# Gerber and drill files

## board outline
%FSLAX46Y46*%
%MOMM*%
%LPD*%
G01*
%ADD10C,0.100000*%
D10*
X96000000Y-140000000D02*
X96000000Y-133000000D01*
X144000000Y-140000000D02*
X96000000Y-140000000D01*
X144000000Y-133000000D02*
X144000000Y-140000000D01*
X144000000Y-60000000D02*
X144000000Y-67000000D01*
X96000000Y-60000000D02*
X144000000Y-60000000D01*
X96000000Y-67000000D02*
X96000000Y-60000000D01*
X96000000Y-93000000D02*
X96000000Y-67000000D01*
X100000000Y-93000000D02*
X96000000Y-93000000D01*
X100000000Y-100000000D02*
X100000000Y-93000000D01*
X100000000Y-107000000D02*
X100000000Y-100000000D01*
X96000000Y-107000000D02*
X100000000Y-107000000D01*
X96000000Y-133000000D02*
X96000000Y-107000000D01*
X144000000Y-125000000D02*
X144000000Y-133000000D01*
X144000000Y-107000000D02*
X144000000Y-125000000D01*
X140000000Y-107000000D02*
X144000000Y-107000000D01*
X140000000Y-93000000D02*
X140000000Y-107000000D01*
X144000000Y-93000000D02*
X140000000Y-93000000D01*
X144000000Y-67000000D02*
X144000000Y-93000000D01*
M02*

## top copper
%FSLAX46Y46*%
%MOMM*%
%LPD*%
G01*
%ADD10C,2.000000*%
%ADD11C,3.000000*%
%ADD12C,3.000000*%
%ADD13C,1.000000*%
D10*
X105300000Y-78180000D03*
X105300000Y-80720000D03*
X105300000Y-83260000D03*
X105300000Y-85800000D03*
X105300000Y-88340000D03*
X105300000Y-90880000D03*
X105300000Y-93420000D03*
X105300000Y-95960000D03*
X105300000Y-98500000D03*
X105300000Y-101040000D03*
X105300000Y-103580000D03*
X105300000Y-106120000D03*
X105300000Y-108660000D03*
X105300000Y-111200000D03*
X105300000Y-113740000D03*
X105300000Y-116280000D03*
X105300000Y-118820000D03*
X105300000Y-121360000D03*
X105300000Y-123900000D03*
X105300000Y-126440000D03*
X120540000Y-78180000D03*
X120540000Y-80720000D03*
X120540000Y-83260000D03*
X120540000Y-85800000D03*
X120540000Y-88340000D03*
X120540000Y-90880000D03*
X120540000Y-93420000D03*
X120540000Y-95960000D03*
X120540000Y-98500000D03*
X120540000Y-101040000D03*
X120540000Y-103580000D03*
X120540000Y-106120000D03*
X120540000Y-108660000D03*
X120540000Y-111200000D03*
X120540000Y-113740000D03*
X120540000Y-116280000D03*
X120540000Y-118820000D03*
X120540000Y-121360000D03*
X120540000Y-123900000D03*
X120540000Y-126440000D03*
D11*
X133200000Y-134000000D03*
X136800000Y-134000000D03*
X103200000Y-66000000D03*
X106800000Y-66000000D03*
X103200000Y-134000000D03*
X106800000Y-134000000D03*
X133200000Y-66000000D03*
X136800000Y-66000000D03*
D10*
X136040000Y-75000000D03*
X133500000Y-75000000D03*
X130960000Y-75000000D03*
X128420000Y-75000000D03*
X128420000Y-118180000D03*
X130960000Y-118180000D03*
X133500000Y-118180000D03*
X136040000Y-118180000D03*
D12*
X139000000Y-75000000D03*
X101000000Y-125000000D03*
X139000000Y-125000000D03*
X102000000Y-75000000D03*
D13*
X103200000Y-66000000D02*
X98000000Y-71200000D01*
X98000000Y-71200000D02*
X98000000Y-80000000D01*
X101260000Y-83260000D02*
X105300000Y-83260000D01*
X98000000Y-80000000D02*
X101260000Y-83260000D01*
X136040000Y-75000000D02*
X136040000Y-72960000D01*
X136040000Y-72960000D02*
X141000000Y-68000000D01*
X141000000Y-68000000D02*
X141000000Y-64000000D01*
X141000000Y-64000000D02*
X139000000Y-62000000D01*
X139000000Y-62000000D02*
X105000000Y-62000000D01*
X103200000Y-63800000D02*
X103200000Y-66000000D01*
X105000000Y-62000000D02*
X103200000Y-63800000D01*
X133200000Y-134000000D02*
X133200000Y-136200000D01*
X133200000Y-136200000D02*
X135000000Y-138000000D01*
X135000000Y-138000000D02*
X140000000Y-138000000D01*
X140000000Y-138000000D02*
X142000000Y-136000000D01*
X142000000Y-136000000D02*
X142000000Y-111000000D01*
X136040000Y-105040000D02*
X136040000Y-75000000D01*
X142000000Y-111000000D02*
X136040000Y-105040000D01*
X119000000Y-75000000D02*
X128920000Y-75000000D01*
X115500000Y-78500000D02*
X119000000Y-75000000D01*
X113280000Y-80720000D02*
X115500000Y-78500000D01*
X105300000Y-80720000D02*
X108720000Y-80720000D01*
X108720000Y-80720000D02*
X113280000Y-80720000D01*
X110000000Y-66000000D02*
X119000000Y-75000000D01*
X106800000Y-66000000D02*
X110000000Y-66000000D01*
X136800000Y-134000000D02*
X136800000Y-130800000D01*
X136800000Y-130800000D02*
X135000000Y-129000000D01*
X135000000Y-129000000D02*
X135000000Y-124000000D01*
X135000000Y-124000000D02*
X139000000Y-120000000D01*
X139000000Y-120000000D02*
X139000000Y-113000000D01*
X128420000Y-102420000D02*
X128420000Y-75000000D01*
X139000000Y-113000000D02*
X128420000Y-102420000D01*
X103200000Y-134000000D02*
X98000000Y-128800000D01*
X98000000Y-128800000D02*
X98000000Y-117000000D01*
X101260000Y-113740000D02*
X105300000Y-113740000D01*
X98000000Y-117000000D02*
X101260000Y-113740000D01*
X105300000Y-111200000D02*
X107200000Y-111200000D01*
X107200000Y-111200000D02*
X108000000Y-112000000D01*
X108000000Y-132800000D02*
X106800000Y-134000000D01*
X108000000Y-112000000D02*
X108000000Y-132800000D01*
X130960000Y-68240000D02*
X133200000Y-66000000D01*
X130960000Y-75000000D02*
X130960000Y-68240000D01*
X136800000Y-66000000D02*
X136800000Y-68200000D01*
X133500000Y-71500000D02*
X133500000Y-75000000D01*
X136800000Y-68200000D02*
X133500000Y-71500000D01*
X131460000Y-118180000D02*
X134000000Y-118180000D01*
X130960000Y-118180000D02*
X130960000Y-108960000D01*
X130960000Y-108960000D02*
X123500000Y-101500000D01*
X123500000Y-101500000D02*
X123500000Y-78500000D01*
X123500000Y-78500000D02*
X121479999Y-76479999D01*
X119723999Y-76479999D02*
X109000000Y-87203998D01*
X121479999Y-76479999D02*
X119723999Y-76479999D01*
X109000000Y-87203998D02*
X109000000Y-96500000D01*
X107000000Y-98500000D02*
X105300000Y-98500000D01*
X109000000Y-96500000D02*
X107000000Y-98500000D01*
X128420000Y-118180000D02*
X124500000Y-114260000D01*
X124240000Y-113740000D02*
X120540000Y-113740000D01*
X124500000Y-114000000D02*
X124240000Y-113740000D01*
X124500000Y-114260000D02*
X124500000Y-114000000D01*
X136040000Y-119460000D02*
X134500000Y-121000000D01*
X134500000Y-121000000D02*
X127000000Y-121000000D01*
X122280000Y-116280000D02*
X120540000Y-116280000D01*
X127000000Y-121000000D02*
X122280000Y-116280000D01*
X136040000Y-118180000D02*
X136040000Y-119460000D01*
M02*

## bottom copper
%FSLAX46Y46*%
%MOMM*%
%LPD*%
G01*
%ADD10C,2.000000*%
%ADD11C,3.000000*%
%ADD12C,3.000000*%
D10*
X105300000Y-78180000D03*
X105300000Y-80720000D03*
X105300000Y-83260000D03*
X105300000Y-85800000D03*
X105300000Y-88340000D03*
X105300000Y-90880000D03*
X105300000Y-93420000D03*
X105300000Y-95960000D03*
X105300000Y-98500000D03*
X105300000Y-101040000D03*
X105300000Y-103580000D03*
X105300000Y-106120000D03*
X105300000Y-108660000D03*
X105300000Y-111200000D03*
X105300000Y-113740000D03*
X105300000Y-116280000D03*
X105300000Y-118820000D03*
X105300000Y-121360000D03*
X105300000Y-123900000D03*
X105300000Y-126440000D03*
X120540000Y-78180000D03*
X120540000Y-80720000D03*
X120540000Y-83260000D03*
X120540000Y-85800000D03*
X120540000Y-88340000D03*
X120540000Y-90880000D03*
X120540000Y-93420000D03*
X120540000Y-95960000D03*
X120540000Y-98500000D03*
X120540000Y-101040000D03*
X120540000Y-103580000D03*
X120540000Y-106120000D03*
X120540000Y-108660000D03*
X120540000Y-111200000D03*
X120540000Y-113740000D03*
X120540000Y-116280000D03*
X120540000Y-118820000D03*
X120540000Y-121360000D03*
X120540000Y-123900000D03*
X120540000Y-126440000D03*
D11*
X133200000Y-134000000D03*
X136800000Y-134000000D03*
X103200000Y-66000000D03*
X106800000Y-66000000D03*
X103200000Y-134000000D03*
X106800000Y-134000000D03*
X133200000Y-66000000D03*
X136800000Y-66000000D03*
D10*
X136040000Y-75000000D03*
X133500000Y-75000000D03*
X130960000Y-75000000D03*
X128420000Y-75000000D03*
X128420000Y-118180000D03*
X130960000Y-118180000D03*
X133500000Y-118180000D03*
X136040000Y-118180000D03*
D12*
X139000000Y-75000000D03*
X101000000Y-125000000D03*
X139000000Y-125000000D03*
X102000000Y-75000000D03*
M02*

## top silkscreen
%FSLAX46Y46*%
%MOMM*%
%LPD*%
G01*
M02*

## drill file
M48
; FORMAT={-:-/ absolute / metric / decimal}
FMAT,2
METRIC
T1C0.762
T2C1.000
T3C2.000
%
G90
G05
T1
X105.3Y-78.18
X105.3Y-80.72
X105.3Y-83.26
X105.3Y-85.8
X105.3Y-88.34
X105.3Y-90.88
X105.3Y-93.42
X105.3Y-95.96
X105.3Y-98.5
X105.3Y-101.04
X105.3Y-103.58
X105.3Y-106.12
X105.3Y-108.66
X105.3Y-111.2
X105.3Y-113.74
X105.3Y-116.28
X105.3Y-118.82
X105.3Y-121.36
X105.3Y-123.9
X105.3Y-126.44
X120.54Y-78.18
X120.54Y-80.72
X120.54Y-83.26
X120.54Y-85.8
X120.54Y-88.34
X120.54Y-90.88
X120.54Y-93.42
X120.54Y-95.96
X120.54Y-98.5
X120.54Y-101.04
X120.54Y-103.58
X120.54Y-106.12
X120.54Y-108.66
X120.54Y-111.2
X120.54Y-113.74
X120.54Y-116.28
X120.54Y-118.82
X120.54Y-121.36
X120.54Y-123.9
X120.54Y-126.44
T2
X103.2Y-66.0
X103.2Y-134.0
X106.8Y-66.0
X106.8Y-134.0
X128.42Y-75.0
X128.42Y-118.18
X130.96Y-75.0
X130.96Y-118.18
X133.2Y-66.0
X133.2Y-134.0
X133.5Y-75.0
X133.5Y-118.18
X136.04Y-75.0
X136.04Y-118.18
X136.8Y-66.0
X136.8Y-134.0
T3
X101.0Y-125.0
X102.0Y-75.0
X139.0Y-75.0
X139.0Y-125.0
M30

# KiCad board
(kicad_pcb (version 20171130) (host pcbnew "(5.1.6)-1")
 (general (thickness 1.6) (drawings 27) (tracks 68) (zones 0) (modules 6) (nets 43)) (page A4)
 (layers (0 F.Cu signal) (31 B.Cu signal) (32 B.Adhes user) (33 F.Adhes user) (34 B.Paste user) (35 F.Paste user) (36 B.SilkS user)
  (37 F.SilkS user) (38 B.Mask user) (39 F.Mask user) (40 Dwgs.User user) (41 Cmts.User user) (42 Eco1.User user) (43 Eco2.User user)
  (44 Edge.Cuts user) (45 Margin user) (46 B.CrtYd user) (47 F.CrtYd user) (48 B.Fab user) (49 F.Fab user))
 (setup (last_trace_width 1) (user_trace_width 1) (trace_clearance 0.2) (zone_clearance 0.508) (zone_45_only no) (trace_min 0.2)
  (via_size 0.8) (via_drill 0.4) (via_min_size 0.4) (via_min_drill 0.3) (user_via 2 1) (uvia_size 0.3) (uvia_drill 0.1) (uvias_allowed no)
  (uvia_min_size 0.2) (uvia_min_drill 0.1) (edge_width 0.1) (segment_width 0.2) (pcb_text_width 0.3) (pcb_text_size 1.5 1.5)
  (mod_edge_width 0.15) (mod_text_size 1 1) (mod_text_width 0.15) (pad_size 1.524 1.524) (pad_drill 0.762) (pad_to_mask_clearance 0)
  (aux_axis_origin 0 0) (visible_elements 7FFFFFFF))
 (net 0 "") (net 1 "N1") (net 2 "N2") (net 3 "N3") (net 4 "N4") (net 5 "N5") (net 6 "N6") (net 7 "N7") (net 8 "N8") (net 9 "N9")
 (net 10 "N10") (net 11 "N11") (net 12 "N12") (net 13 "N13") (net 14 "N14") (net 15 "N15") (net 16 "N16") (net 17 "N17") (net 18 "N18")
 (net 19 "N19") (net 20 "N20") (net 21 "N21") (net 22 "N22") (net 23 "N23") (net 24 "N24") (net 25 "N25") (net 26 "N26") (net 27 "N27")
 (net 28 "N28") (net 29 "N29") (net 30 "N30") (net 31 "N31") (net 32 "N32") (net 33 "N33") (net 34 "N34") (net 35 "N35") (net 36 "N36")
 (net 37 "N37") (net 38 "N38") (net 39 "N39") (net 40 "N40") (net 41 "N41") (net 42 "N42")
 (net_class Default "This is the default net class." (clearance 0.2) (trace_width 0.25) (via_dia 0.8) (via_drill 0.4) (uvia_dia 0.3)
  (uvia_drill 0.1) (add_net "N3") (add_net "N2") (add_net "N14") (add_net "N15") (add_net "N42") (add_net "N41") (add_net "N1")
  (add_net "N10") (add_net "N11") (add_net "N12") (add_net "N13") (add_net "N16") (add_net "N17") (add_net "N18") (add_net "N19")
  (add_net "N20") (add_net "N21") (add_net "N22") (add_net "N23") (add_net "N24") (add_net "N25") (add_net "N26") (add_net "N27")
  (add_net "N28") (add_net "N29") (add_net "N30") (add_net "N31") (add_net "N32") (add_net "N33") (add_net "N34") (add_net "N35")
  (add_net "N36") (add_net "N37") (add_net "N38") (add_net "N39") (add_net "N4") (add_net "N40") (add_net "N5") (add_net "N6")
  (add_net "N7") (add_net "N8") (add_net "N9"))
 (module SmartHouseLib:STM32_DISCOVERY (layer B.Cu) (at 118 98.5 180)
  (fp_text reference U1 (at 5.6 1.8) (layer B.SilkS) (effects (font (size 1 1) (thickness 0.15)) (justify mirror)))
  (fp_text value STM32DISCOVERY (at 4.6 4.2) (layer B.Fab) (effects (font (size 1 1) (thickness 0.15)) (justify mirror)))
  (pad 1 thru_hole circle (at 12.7 20.32 180) (size 2 2) (drill 0.762) (layers *.Cu *.Mask) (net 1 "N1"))
  (pad 2 thru_hole circle (at 12.7 17.78 180) (size 2 2) (drill 0.762) (layers *.Cu *.Mask) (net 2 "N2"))
  (pad 3 thru_hole circle (at 12.7 15.24 180) (size 2 2) (drill 0.762) (layers *.Cu *.Mask) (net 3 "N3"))
  (pad 4 thru_hole circle (at 12.7 12.7 180) (size 2 2) (drill 0.762) (layers *.Cu *.Mask) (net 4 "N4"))
  (pad 5 thru_hole circle (at 12.7 10.16 180) (size 2 2) (drill 0.762) (layers *.Cu *.Mask) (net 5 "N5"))
  (pad 6 thru_hole circle (at 12.7 7.62 180) (size 2 2) (drill 0.762) (layers *.Cu *.Mask) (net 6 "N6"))
  (pad 7 thru_hole circle (at 12.7 5.08 180) (size 2 2) (drill 0.762) (layers *.Cu *.Mask) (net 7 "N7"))
  (pad 8 thru_hole circle (at 12.7 2.54 180) (size 2 2) (drill 0.762) (layers *.Cu *.Mask) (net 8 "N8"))
  (pad 9 thru_hole circle (at 12.7 0 180) (size 2 2) (drill 0.762) (layers *.Cu *.Mask) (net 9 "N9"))
  (pad 10 thru_hole circle (at 12.7 -2.54 180) (size 2 2) (drill 0.762) (layers *.Cu *.Mask) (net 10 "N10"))
  (pad 11 thru_hole circle (at 12.7 -5.08 180) (size 2 2) (drill 0.762) (layers *.Cu *.Mask) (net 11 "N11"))
  (pad 12 thru_hole circle (at 12.7 -7.62 180) (size 2 2) (drill 0.762) (layers *.Cu *.Mask) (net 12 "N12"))
  (pad 13 thru_hole circle (at 12.7 -10.16 180) (size 2 2) (drill 0.762) (layers *.Cu *.Mask) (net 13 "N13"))
  (pad 14 thru_hole circle (at 12.7 -12.7 180) (size 2 2) (drill 0.762) (layers *.Cu *.Mask) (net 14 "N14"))
  (pad 15 thru_hole circle (at 12.7 -15.24 180) (size 2 2) (drill 0.762) (layers *.Cu *.Mask) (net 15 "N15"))
  (pad 16 thru_hole circle (at 12.7 -17.78 180) (size 2 2) (drill 0.762) (layers *.Cu *.Mask) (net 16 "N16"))
  (pad 17 thru_hole circle (at 12.7 -20.32 180) (size 2 2) (drill 0.762) (layers *.Cu *.Mask) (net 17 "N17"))
  (pad 18 thru_hole circle (at 12.7 -22.86 180) (size 2 2) (drill 0.762) (layers *.Cu *.Mask) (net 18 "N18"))
  (pad 19 thru_hole circle (at 12.7 -25.4 180) (size 2 2) (drill 0.762) (layers *.Cu *.Mask) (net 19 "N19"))
  (pad 20 thru_hole circle (at 12.7 -27.94 180) (size 2 2) (drill 0.762) (layers *.Cu *.Mask) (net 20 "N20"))
  (pad 21 thru_hole circle (at -2.54 20.32 180) (size 2 2) (drill 0.762) (layers *.Cu *.Mask) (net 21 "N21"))
  (pad 22 thru_hole circle (at -2.54 17.78 180) (size 2 2) (drill 0.762) (layers *.Cu *.Mask) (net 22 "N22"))
  (pad 23 thru_hole circle (at -2.54 15.24 180) (size 2 2) (drill 0.762) (layers *.Cu *.Mask) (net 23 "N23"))
  (pad 24 thru_hole circle (at -2.54 12.7 180) (size 2 2) (drill 0.762) (layers *.Cu *.Mask) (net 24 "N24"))
  (pad 25 thru_hole circle (at -2.54 10.16 180) (size 2 2) (drill 0.762) (layers *.Cu *.Mask) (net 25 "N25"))
  (pad 26 thru_hole circle (at -2.54 7.62 180) (size 2 2) (drill 0.762) (layers *.Cu *.Mask) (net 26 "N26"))
  (pad 27 thru_hole circle (at -2.54 5.08 180) (size 2 2) (drill 0.762) (layers *.Cu *.Mask) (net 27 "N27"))
  (pad 28 thru_hole circle (at -2.54 2.54 180) (size 2 2) (drill 0.762) (layers *.Cu *.Mask) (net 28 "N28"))
  (pad 29 thru_hole circle (at -2.54 0 180) (size 2 2) (drill 0.762) (layers *.Cu *.Mask) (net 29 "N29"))
  (pad 30 thru_hole circle (at -2.54 -2.54 180) (size 2 2) (drill 0.762) (layers *.Cu *.Mask) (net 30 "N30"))
  (pad 31 thru_hole circle (at -2.54 -5.08 180) (size 2 2) (drill 0.762) (layers *.Cu *.Mask) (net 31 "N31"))
  (pad 32 thru_hole circle (at -2.54 -7.62 180) (size 2 2) (drill 0.762) (layers *.Cu *.Mask) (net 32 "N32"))
  (pad 33 thru_hole circle (at -2.54 -10.16 180) (size 2 2) (drill 0.762) (layers *.Cu *.Mask) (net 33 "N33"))
  (pad 34 thru_hole circle (at -2.54 -12.7 180) (size 2 2) (drill 0.762) (layers *.Cu *.Mask) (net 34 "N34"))
  (pad 35 thru_hole circle (at -2.54 -15.24 180) (size 2 2) (drill 0.762) (layers *.Cu *.Mask) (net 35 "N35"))
  (pad 36 thru_hole circle (at -2.54 -17.78 180) (size 2 2) (drill 0.762) (layers *.Cu *.Mask) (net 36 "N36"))
  (pad 37 thru_hole circle (at -2.54 -20.32 180) (size 2 2) (drill 0.762) (layers *.Cu *.Mask) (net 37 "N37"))
  (pad 38 thru_hole circle (at -2.54 -22.86 180) (size 2 2) (drill 0.762) (layers *.Cu *.Mask) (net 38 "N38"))
  (pad 39 thru_hole circle (at -2.54 -25.4 180) (size 2 2) (drill 0.762) (layers *.Cu *.Mask) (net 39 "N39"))
  (pad 40 thru_hole circle (at -2.54 -27.94 180) (size 2 2) (drill 0.762) (layers *.Cu *.Mask) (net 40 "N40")))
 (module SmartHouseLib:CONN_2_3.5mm (layer B.Cu) (at 135 134)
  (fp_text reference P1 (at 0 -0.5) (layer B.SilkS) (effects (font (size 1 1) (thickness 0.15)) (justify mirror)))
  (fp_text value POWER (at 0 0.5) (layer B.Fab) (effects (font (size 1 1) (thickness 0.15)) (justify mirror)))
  (pad 1 thru_hole circle (at -1.8 0) (size 3 3) (drill 1) (layers *.Cu *.Mask) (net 3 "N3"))
  (pad 2 thru_hole circle (at 1.8 0) (size 3 3) (drill 1) (layers *.Cu *.Mask) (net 2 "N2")))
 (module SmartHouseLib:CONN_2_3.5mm (layer B.Cu) (at 105 66)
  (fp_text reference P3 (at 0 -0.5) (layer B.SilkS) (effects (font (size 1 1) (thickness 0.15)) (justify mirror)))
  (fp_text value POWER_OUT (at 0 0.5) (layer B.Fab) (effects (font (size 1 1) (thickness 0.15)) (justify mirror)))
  (pad 1 thru_hole circle (at -1.8 0) (size 3 3) (drill 1) (layers *.Cu *.Mask) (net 3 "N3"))
  (pad 2 thru_hole circle (at 1.8 0) (size 3 3) (drill 1) (layers *.Cu *.Mask) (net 2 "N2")))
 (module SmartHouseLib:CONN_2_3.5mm (layer B.Cu) (at 105 134 180)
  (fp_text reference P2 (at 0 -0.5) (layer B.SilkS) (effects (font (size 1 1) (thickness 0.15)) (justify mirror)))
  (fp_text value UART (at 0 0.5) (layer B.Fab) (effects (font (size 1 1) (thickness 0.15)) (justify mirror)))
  (pad 2 thru_hole circle (at 1.8 0 180) (size 3 3) (drill 1) (layers *.Cu *.Mask) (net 15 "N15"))
  (pad 1 thru_hole circle (at -1.8 0 180) (size 3 3) (drill 1) (layers *.Cu *.Mask) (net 14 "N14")))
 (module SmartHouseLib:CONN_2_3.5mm (layer B.Cu) (at 135 66 180)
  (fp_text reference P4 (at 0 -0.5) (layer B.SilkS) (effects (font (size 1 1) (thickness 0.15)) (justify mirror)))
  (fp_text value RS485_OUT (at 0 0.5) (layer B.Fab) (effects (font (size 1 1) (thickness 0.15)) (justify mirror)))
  (pad 2 thru_hole circle (at 1.8 0 180) (size 3 3) (drill 1) (layers *.Cu *.Mask) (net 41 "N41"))
  (pad 1 thru_hole circle (at -1.8 0 180) (size 3 3) (drill 1) (layers *.Cu *.Mask) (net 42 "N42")))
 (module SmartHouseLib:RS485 (layer B.Cu) (at 133.5 75 180)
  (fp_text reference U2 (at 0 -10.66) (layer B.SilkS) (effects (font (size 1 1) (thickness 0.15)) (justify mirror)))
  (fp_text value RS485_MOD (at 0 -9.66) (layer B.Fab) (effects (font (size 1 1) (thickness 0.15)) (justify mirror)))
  (pad 1 thru_hole circle (at -2.54 0 180) (size 2 2) (drill 1) (layers *.Cu *.Mask) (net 3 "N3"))
  (pad 2 thru_hole circle (at 0 0 180) (size 2 2) (drill 1) (layers *.Cu *.Mask) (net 42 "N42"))
  (pad 3 thru_hole circle (at 2.54 0 180) (size 2 2) (drill 1) (layers *.Cu *.Mask) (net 41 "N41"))
  (pad 4 thru_hole circle (at 5.08 0 180) (size 2 2) (drill 1) (layers *.Cu *.Mask) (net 2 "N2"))
  (pad 5 thru_hole circle (at 5.08 -43.18 180) (size 2 2) (drill 1) (layers *.Cu *.Mask) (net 35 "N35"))
  (pad 6 thru_hole circle (at 2.54 -43.18 180) (size 2 2) (drill 1) (layers *.Cu *.Mask) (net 9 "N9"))
  (pad 7 thru_hole circle (at 0 -43.18 180) (size 2 2) (drill 1) (layers *.Cu *.Mask) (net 9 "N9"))
  (pad 8 thru_hole circle (at -2.54 -43.18 180) (size 2 2) (drill 1) (layers *.Cu *.Mask) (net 36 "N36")))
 (gr_line (start 96 140) (end 96 133) (layer Edge.Cuts) (width 0.1))
 (gr_line (start 144 140) (end 96 140) (layer Edge.Cuts) (width 0.1))
 (gr_line (start 144 133) (end 144 140) (layer Edge.Cuts) (width 0.1))
 (gr_line (start 144 60) (end 144 67) (layer Edge.Cuts) (width 0.1))
 (gr_line (start 96 60) (end 144 60) (layer Edge.Cuts) (width 0.1))
 (gr_line (start 96 67) (end 96 60) (layer Edge.Cuts) (width 0.1))
 (gr_line (start 96 93) (end 96 67) (layer Edge.Cuts) (width 0.1))
 (gr_line (start 100 93) (end 96 93) (layer Edge.Cuts) (width 0.1))
 (gr_line (start 100 100) (end 100 93) (layer Edge.Cuts) (width 0.1))
 (gr_line (start 100 107) (end 100 100) (layer Edge.Cuts) (width 0.1))
 (gr_line (start 96 107) (end 100 107) (layer Edge.Cuts) (width 0.1))
 (gr_line (start 96 133) (end 96 107) (layer Edge.Cuts) (width 0.1))
 (gr_line (start 144 125) (end 144 133) (layer Edge.Cuts) (width 0.1))
 (gr_line (start 144 107) (end 144 125) (layer Edge.Cuts) (width 0.1))
 (gr_line (start 140 107) (end 144 107) (layer Edge.Cuts) (width 0.1))
 (gr_line (start 140 93) (end 140 107) (layer Edge.Cuts) (width 0.1))
 (gr_line (start 144 93) (end 140 93) (layer Edge.Cuts) (width 0.1))
 (gr_line (start 144 67) (end 144 93) (layer Edge.Cuts) (width 0.1))
 (via (at 139 75) (size 3) (drill 2) (layers F.Cu B.Cu) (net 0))
 (via (at 101 125) (size 3) (drill 2) (layers F.Cu B.Cu) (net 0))
 (via (at 139 125) (size 3) (drill 2) (layers F.Cu B.Cu) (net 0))
 (segment (start 103.2 66) (end 98 71.2) (width 1) (layer F.Cu) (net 3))
 (segment (start 98 71.2) (end 98 80) (width 1) (layer F.Cu) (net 3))
 (segment (start 101.26 83.26) (end 105.3 83.26) (width 1) (layer F.Cu) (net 3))
 (segment (start 98 80) (end 101.26 83.26) (width 1) (layer F.Cu) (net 3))
 (segment (start 136.04 75) (end 136.04 72.96) (width 1) (layer F.Cu) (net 3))
 (segment (start 136.04 72.96) (end 141 68) (width 1) (layer F.Cu) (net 3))
 (segment (start 141 68) (end 141 64) (width 1) (layer F.Cu) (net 3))
 (segment (start 141 64) (end 139 62) (width 1) (layer F.Cu) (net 3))
 (segment (start 139 62) (end 105 62) (width 1) (layer F.Cu) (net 3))
 (segment (start 103.2 63.8) (end 103.2 66) (width 1) (layer F.Cu) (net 3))
 (segment (start 105 62) (end 103.2 63.8) (width 1) (layer F.Cu) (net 3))
 (segment (start 133.2 134) (end 133.2 136.2) (width 1) (layer F.Cu) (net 3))
 (segment (start 133.2 136.2) (end 135 138) (width 1) (layer F.Cu) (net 3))
 (segment (start 135 138) (end 140 138) (width 1) (layer F.Cu) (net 3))
 (segment (start 140 138) (end 142 136) (width 1) (layer F.Cu) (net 3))
 (segment (start 142 136) (end 142 111) (width 1) (layer F.Cu) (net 3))
 (segment (start 136.04 105.04) (end 136.04 75) (width 1) (layer F.Cu) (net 3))
 (segment (start 142 111) (end 136.04 105.04) (width 1) (layer F.Cu) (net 3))
 (segment (start 119 75) (end 128.92 75) (width 1) (layer F.Cu) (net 2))
 (segment (start 115.5 78.5) (end 119 75) (width 1) (layer F.Cu) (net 2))
 (segment (start 113.28 80.72) (end 115.5 78.5) (width 1) (layer F.Cu) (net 2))
 (segment (start 105.3 80.72) (end 108.72 80.72) (width 1) (layer F.Cu) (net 2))
 (segment (start 108.72 80.72) (end 113.28 80.72) (width 1) (layer F.Cu) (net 2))
 (segment (start 110 66) (end 119 75) (width 1) (layer F.Cu) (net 2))
 (segment (start 106.8 66) (end 110 66) (width 1) (layer F.Cu) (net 2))
 (segment (start 136.8 134) (end 136.8 130.8) (width 1) (layer F.Cu) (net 2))
 (segment (start 136.8 130.8) (end 135 129) (width 1) (layer F.Cu) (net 2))
 (segment (start 135 129) (end 135 124) (width 1) (layer F.Cu) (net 2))
 (segment (start 135 124) (end 139 120) (width 1) (layer F.Cu) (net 2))
 (segment (start 139 120) (end 139 113) (width 1) (layer F.Cu) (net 2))
 (segment (start 128.42 102.42) (end 128.42 75) (width 1) (layer F.Cu) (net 2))
 (segment (start 139 113) (end 128.42 102.42) (width 1) (layer F.Cu) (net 2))
 (segment (start 103.2 134) (end 98 128.8) (width 1) (layer F.Cu) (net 15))
 (segment (start 98 128.8) (end 98 117) (width 1) (layer F.Cu) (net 15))
 (segment (start 101.26 113.74) (end 105.3 113.74) (width 1) (layer F.Cu) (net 15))
 (segment (start 98 117) (end 101.26 113.74) (width 1) (layer F.Cu) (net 15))
 (segment (start 105.3 111.2) (end 107.2 111.2) (width 1) (layer F.Cu) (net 14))
 (segment (start 107.2 111.2) (end 108 112) (width 1) (layer F.Cu) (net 14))
 (segment (start 108 132.8) (end 106.8 134) (width 1) (layer F.Cu) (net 14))
 (segment (start 108 112) (end 108 132.8) (width 1) (layer F.Cu) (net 14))
 (segment (start 130.96 68.24) (end 133.2 66) (width 1) (layer F.Cu) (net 41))
 (segment (start 130.96 75) (end 130.96 68.24) (width 1) (layer F.Cu) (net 41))
 (segment (start 136.8 66) (end 136.8 68.2) (width 1) (layer F.Cu) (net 42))
 (segment (start 133.5 71.5) (end 133.5 75) (width 1) (layer F.Cu) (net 42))
 (segment (start 136.8 68.2) (end 133.5 71.5) (width 1) (layer F.Cu) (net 42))
 (segment (start 131.46 118.18) (end 134 118.18) (width 1) (layer F.Cu) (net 9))
 (segment (start 130.96 118.18) (end 130.96 108.96) (width 1) (layer F.Cu) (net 9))
 (segment (start 130.96 108.96) (end 123.5 101.5) (width 1) (layer F.Cu) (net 9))
 (segment (start 123.5 101.5) (end 123.5 78.5) (width 1) (layer F.Cu) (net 9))
 (segment (start 123.5 78.5) (end 121.479999 76.479999) (width 1) (layer F.Cu) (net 9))
 (segment (start 119.723999 76.479999) (end 109 87.203998) (width 1) (layer F.Cu) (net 9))
 (segment (start 121.479999 76.479999) (end 119.723999 76.479999) (width 1) (layer F.Cu) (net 9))
 (segment (start 109 87.203998) (end 109 96.5) (width 1) (layer F.Cu) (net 9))
 (segment (start 107 98.5) (end 105.3 98.5) (width 1) (layer F.Cu) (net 9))
 (segment (start 109 96.5) (end 107 98.5) (width 1) (layer F.Cu) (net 9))
 (segment (start 128.42 118.18) (end 124.5 114.26) (width 1) (layer F.Cu) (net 35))
 (segment (start 124.24 113.74) (end 120.54 113.74) (width 1) (layer F.Cu) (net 35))
 (segment (start 124.5 114) (end 124.24 113.74) (width 1) (layer F.Cu) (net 35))
 (segment (start 124.5 114.26) (end 124.5 114) (width 1) (layer F.Cu) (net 35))
 (via (at 102 75) (size 3) (drill 2) (layers F.Cu B.Cu) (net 36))
 (segment (start 136.04 119.46) (end 134.5 121) (width 1) (layer F.Cu) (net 36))
 (segment (start 134.5 121) (end 127 121) (width 1) (layer F.Cu) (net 36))
 (segment (start 122.28 116.28) (end 120.54 116.28) (width 1) (layer F.Cu) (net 36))
 (segment (start 127 121) (end 122.28 116.28) (width 1) (layer F.Cu) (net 36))
 (segment (start 136.04 118.18) (end 136.04 119.46) (width 1) (layer F.Cu) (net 36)))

